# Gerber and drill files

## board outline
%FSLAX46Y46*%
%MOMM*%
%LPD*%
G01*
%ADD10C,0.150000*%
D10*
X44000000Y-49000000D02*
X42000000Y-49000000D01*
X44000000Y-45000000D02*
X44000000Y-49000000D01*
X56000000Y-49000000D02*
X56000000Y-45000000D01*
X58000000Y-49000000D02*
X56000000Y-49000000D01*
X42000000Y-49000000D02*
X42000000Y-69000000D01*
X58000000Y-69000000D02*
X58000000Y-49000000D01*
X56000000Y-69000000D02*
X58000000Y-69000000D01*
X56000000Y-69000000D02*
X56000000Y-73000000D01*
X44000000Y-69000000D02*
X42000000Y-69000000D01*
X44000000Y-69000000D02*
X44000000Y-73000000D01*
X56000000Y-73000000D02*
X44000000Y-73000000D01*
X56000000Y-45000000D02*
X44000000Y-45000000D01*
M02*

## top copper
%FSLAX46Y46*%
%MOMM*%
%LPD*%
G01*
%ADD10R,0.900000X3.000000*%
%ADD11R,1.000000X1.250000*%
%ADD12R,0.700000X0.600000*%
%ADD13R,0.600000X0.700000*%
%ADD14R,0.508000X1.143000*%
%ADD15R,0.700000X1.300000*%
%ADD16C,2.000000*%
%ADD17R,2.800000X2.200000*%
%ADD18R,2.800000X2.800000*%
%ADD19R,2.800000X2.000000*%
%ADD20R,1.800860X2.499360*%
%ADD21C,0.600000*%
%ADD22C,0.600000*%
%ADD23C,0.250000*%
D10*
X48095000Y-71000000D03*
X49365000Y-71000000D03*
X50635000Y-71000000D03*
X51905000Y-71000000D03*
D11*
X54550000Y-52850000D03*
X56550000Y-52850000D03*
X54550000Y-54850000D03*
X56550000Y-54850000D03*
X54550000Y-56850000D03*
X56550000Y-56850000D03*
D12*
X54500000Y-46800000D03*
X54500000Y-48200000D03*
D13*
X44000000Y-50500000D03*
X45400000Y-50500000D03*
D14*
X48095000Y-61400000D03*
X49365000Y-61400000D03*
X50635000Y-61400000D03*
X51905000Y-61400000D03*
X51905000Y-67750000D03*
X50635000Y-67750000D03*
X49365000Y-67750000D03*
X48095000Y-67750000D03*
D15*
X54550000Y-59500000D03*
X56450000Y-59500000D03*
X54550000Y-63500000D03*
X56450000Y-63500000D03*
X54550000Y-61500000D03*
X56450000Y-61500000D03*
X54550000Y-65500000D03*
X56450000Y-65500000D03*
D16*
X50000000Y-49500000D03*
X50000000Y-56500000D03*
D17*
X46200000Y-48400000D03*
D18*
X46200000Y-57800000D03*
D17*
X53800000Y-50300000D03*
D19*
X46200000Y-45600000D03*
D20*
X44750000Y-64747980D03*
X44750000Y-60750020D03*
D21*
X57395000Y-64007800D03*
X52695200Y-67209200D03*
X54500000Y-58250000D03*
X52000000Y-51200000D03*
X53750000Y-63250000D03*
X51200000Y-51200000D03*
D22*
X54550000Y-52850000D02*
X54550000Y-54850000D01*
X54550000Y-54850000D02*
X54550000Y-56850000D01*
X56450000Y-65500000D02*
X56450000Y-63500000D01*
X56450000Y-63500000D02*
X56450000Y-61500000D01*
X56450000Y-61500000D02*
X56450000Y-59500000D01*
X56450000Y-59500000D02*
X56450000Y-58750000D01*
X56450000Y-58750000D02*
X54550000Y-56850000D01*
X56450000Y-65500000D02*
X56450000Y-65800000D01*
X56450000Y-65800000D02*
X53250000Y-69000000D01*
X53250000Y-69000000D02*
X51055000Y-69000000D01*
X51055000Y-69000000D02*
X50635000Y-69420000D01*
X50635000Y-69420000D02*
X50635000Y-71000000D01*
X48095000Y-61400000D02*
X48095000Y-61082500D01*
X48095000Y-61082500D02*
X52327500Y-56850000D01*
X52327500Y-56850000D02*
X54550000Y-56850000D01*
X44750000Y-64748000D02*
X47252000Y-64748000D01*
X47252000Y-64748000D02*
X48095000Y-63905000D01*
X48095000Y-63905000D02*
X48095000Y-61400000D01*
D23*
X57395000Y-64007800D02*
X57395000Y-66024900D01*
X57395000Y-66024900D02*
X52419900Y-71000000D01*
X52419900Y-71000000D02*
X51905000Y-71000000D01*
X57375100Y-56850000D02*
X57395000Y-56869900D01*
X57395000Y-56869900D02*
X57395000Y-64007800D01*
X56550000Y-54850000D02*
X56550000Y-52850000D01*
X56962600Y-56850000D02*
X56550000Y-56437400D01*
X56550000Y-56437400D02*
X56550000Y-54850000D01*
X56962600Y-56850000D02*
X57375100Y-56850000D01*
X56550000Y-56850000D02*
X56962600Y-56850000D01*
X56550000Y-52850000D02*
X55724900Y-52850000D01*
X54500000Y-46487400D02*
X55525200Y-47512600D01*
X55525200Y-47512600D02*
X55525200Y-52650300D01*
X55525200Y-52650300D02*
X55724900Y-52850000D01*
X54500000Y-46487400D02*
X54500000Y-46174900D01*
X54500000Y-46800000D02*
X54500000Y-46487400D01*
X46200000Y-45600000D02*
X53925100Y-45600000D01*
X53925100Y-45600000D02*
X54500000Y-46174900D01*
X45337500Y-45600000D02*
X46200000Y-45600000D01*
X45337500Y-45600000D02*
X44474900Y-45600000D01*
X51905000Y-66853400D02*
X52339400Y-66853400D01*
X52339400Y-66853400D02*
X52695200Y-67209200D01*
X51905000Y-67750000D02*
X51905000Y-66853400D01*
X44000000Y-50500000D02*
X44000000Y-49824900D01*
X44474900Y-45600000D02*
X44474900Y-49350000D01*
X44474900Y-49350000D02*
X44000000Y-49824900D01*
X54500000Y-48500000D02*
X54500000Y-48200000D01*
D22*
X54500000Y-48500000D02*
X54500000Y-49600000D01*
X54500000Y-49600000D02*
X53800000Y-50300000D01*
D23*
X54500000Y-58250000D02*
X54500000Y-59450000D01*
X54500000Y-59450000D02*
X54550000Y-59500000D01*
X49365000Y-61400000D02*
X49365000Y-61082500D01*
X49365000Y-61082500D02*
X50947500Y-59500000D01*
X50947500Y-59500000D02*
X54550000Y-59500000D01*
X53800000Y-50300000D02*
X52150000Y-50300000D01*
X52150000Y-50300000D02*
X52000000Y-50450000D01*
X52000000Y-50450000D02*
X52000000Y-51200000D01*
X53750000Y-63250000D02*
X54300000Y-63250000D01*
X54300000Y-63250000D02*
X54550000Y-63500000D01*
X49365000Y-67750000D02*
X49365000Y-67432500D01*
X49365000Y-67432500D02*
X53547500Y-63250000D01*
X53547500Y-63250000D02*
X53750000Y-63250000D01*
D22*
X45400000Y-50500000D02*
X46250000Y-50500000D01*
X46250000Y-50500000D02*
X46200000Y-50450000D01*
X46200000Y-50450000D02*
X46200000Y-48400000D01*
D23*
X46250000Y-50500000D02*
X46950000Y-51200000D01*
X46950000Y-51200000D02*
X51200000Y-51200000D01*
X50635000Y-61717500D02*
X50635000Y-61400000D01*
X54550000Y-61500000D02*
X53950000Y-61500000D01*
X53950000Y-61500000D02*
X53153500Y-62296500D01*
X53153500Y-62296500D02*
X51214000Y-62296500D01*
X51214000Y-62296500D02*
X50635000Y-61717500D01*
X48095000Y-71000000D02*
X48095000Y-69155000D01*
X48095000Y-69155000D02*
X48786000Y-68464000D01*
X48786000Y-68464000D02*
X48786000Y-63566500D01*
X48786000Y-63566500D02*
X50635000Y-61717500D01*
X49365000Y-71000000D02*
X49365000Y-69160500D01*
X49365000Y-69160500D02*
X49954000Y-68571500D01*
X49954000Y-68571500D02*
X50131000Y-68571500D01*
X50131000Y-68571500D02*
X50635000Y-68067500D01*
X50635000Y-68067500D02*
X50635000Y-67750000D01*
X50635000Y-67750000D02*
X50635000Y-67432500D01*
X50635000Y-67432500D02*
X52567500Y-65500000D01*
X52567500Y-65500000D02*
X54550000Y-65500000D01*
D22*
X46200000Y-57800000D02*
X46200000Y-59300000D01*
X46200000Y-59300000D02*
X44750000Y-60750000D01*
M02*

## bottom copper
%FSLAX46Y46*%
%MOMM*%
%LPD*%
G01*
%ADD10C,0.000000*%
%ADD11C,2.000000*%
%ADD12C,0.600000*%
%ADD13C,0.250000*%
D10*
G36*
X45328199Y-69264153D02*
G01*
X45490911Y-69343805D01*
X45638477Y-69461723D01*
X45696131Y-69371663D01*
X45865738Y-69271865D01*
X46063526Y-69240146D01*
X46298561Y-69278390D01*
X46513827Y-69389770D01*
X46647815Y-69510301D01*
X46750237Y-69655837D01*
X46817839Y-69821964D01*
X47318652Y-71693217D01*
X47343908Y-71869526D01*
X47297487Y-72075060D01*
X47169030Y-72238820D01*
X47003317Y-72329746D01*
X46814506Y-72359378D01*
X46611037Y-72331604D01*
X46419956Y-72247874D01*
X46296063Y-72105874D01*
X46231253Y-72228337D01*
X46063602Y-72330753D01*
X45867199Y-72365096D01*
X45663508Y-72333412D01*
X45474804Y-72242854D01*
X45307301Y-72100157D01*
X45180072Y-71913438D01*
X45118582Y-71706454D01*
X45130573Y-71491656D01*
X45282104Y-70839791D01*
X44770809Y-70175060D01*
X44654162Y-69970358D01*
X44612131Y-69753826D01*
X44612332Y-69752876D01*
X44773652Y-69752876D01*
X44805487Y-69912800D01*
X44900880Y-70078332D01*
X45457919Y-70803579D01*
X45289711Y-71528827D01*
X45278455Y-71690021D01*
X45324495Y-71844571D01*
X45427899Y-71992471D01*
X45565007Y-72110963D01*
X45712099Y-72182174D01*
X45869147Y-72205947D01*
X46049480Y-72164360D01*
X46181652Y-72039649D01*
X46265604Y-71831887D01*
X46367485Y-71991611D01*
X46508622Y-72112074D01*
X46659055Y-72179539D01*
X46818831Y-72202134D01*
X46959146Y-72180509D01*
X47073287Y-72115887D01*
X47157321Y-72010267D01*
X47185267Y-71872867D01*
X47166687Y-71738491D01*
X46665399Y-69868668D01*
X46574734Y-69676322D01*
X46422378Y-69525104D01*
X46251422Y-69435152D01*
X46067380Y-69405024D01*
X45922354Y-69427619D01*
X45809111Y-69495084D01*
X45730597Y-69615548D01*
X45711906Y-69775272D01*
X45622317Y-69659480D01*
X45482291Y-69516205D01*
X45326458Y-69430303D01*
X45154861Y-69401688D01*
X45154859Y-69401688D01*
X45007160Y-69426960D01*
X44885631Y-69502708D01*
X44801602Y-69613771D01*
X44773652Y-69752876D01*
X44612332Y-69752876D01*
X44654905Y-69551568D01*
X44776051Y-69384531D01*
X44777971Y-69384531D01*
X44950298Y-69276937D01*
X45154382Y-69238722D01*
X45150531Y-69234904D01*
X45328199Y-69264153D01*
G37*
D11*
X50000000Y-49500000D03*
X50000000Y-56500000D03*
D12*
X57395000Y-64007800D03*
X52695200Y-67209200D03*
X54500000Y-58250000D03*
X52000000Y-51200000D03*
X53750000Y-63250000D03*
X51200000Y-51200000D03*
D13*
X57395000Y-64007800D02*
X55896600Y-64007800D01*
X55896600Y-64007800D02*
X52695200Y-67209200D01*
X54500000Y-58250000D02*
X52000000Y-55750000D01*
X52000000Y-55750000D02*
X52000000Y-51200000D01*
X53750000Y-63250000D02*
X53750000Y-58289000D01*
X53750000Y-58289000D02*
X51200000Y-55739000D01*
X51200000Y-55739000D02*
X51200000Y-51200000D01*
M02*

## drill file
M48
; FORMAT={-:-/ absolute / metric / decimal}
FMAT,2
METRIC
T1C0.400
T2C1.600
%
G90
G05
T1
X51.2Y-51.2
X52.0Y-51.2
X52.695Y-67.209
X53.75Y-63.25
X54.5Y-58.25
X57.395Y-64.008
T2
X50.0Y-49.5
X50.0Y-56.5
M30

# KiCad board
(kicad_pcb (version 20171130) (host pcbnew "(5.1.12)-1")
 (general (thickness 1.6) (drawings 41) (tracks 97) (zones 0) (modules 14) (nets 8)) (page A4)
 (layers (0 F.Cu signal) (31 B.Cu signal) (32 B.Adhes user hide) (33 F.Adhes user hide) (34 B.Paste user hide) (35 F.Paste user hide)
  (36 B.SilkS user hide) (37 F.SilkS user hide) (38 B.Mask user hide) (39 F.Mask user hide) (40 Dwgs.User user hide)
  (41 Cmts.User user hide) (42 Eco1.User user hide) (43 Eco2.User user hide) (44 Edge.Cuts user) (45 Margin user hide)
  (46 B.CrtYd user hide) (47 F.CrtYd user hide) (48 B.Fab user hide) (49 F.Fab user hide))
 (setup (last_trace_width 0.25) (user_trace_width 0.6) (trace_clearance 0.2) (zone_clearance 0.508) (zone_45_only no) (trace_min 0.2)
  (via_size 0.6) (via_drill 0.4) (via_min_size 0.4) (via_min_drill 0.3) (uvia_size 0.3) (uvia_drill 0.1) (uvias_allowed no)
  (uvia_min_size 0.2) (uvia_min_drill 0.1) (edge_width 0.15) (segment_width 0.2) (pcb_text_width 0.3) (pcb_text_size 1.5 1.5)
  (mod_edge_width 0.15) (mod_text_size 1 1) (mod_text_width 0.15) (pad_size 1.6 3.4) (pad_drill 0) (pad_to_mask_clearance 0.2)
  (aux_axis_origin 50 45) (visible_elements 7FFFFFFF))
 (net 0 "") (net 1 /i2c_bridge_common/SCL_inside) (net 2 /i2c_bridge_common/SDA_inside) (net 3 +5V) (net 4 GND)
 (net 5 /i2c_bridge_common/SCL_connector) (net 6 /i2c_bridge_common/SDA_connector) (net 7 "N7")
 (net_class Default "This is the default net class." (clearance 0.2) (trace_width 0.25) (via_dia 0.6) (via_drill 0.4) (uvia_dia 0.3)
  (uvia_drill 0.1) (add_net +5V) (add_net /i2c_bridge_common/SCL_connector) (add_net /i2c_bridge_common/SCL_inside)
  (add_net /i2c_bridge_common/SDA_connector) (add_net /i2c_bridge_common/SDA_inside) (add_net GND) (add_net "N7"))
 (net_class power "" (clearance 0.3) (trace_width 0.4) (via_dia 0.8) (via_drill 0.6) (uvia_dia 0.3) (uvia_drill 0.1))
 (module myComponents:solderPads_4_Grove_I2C (layer F.Cu) (at 50 71)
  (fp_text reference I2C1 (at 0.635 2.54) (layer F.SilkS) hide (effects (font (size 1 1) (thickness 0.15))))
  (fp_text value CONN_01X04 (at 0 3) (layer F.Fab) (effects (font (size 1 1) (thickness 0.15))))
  (pad 1 smd rect (at -1.905 0) (size 0.9 3) (layers F.Cu F.Paste F.Mask) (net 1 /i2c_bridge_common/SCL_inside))
  (pad 2 smd rect (at -0.635 0) (size 0.9 3) (layers F.Cu F.Paste F.Mask) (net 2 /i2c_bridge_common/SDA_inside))
  (pad 3 smd rect (at 0.635 0) (size 0.9 3) (layers F.Cu F.Paste F.Mask) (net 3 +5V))
  (pad 4 smd rect (at 1.905 0) (size 0.9 3) (layers F.Cu F.Paste F.Mask) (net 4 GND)))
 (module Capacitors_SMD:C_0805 (layer F.Cu) (at 55.55 52.85)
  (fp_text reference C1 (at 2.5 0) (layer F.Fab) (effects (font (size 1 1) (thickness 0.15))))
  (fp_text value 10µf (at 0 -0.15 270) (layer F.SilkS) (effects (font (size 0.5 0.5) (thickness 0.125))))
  (pad 1 smd rect (at -1 0) (size 1 1.25) (layers F.Cu F.Paste F.Mask) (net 3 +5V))
  (pad 2 smd rect (at 1 0) (size 1 1.25) (layers F.Cu F.Paste F.Mask) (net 4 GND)))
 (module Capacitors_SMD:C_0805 (layer F.Cu) (at 55.55 54.85)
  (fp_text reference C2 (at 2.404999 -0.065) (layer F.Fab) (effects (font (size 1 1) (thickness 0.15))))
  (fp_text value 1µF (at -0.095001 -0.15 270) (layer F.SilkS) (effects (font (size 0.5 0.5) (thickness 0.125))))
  (pad 1 smd rect (at -1 0) (size 1 1.25) (layers F.Cu F.Paste F.Mask) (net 3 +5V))
  (pad 2 smd rect (at 1 0) (size 1 1.25) (layers F.Cu F.Paste F.Mask) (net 4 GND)))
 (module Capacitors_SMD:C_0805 (layer F.Cu) (at 55.55 56.85)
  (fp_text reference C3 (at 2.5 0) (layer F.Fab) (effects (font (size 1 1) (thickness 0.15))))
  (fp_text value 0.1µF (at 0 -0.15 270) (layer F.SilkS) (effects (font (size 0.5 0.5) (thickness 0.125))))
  (pad 1 smd rect (at -1 0) (size 1 1.25) (layers F.Cu F.Paste F.Mask) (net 3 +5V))
  (pad 2 smd rect (at 1 0) (size 1 1.25) (layers F.Cu F.Paste F.Mask) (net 4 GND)))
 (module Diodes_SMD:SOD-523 (layer F.Cu) (at 54.5 47.5 90)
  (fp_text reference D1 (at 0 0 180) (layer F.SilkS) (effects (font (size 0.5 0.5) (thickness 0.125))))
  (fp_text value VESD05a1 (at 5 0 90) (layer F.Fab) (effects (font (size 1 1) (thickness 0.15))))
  (pad 2 smd rect (at 0.7 0 270) (size 0.6 0.7) (layers F.Cu F.Paste F.Mask) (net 4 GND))
  (pad 1 smd rect (at -0.7 0 270) (size 0.6 0.7) (layers F.Cu F.Paste F.Mask) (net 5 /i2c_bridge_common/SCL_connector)))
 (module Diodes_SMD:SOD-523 (layer F.Cu) (at 44.7 50.5 180)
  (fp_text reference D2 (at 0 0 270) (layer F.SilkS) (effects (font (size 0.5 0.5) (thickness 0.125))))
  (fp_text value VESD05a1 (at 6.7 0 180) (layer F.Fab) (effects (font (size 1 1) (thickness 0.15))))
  (pad 2 smd rect (at 0.7 0) (size 0.6 0.7) (layers F.Cu F.Paste F.Mask) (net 4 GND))
  (pad 1 smd rect (at -0.7 0) (size 0.6 0.7) (layers F.Cu F.Paste F.Mask) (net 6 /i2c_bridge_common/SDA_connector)))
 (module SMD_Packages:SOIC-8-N (layer F.Cu) (at 50 64.575)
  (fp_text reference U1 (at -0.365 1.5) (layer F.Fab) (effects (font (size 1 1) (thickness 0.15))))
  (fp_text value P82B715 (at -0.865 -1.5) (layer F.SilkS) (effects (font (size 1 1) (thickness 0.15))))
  (pad 8 smd rect (at -1.905 -3.175) (size 0.508 1.143) (layers F.Cu F.Paste F.Mask) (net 3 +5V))
  (pad 7 smd rect (at -0.635 -3.175) (size 0.508 1.143) (layers F.Cu F.Paste F.Mask) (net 5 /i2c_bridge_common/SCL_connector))
  (pad 6 smd rect (at 0.635 -3.175) (size 0.508 1.143) (layers F.Cu F.Paste F.Mask) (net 1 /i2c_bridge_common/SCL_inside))
  (pad 5 smd rect (at 1.905 -3.175) (size 0.508 1.143) (layers F.Cu F.Paste F.Mask))
  (pad 4 smd rect (at 1.905 3.175) (size 0.508 1.143) (layers F.Cu F.Paste F.Mask) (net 4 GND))
  (pad 3 smd rect (at 0.635 3.175) (size 0.508 1.143) (layers F.Cu F.Paste F.Mask) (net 2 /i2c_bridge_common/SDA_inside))
  (pad 2 smd rect (at -0.635 3.175) (size 0.508 1.143) (layers F.Cu F.Paste F.Mask) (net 6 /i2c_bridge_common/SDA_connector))
  (pad 1 smd rect (at -1.905 3.175) (size 0.508 1.143) (layers F.Cu F.Paste F.Mask)))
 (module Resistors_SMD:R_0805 (layer F.Cu) (at 55.5 59.5)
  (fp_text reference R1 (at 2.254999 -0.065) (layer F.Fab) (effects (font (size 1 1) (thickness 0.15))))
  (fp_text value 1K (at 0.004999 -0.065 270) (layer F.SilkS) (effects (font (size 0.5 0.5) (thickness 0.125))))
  (pad 1 smd rect (at -0.95 0) (size 0.7 1.3) (layers F.Cu F.Paste F.Mask) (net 5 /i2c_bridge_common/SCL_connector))
  (pad 2 smd rect (at 0.95 0) (size 0.7 1.3) (layers F.Cu F.Paste F.Mask) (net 3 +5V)))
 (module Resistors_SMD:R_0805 (layer F.Cu) (at 55.5 63.5)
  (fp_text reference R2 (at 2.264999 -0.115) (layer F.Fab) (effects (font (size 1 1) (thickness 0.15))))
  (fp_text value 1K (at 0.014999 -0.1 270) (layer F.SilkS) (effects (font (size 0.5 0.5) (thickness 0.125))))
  (pad 1 smd rect (at -0.95 0) (size 0.7 1.3) (layers F.Cu F.Paste F.Mask) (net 6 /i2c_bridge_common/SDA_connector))
  (pad 2 smd rect (at 0.95 0) (size 0.7 1.3) (layers F.Cu F.Paste F.Mask) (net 3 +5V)))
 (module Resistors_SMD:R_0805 (layer F.Cu) (at 55.5 61.5)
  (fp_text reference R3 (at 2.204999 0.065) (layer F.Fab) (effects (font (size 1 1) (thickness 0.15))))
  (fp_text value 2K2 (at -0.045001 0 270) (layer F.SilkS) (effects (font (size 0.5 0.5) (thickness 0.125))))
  (pad 1 smd rect (at -0.95 0) (size 0.7 1.3) (layers F.Cu F.Paste F.Mask) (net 1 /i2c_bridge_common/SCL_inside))
  (pad 2 smd rect (at 0.95 0) (size 0.7 1.3) (layers F.Cu F.Paste F.Mask) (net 3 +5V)))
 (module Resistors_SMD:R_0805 (layer F.Cu) (at 55.5 65.5)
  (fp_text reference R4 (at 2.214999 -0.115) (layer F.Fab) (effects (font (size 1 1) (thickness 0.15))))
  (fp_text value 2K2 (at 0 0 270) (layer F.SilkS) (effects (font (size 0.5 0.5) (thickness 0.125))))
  (pad 1 smd rect (at -0.95 0) (size 0.7 1.3) (layers F.Cu F.Paste F.Mask) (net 2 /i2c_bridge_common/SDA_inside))
  (pad 2 smd rect (at 0.95 0) (size 0.7 1.3) (layers F.Cu F.Paste F.Mask) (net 3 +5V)))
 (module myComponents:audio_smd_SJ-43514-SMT (layer F.Cu) (at 50 45 270)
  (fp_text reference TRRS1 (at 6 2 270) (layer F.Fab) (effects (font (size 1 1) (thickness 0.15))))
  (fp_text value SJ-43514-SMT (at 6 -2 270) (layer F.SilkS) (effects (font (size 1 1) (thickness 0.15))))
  (pad "" thru_hole circle (at 4.5 0 270) (size 2 2) (drill 1.6) (layers *.Cu *.Mask F.SilkS))
  (pad "" thru_hole circle (at 11.5 0 270) (size 2 2) (drill 1.6) (layers *.Cu *.Mask F.SilkS))
  (pad 4 smd rect (at 3.4 3.8 270) (size 2.2 2.8) (layers F.Cu F.Paste F.Mask) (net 6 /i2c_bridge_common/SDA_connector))
  (pad 2 smd rect (at 12.8 3.8 270) (size 2.8 2.8) (layers F.Cu F.Paste F.Mask) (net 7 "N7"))
  (pad 3 smd rect (at 5.3 -3.8 270) (size 2.2 2.8) (layers F.Cu F.Paste F.Mask) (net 5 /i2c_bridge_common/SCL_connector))
  (pad 1 smd rect (at 0.6 3.8 270) (size 2 2.8) (layers F.Cu F.Paste F.Mask) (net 4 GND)))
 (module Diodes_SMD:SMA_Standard (layer F.Cu) (at 44.75 62.749 90)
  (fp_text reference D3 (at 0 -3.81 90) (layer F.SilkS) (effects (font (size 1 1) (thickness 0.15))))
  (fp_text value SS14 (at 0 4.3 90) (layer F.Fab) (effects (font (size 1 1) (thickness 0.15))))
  (pad 1 smd rect (at -1.99898 0 90) (size 2.49936 1.80086) (layers F.Cu F.Paste F.Mask) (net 3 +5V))
  (pad 2 smd rect (at 1.99898 0 90) (size 2.49936 1.80086) (layers F.Cu F.Paste F.Mask) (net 7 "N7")))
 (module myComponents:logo (layer B.Cu) (at 50 70.8 180)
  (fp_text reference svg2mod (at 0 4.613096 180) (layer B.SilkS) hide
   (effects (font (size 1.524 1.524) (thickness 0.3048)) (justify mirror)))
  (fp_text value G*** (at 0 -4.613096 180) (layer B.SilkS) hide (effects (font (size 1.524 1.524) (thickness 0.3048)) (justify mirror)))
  (fp_poly
   (pts (xy 4.849469 1.565096) (xy 4.269403 1.184452) (xy 4.288094 1.024728) (xy 4.377683 1.14052) (xy 4.517709 1.283795)
    (xy 4.673542 1.369697) (xy 4.845139 1.398312) (xy 4.845141 1.398312) (xy 4.99284 1.37304) (xy 5.114369 1.297292) (xy 5.198398 1.186229)
    (xy 5.226348 1.047124) (xy 5.194513 0.8872) (xy 5.09912 0.721668) (xy 4.542081 -0.003579) (xy 4.710289 -0.728827)
    (xy 4.721545 -0.890021) (xy 4.675505 -1.044571) (xy 4.572101 -1.192471) (xy 4.434993 -1.310963) (xy 4.287901 -1.382174)
    (xy 4.130853 -1.405947) (xy 3.95052 -1.36436) (xy 3.818348 -1.239649) (xy 3.734396 -1.031887) (xy 3.632515 -1.191611)
    (xy 3.491378 -1.312074) (xy 3.340945 -1.379539) (xy 3.181169 -1.402134) (xy 3.040854 -1.380509) (xy 2.926713 -1.315887)
    (xy 2.842679 -1.210267) (xy 2.814733 -1.072867) (xy 2.833313 -0.938491) (xy 3.334601 0.931332) (xy 3.425266 1.123678)
    (xy 3.577622 1.274896) (xy 3.748578 1.364848) (xy 3.93262 1.394976) (xy 4.077646 1.372381) (xy 4.190889 1.304916) (xy 4.269403 1.184452)
    (xy 4.849469 1.565096) (xy 4.671801 1.535847) (xy 4.509089 1.456195) (xy 4.361523 1.338277) (xy 4.303869 1.428337)
    (xy 4.134262 1.528135) (xy 3.936474 1.559854) (xy 3.701439 1.52161) (xy 3.486173 1.41023) (xy 3.352185 1.289699) (xy 3.249763 1.144163)
    (xy 3.182161 0.978036) (xy 2.681348 -0.893217) (xy 2.656092 -1.069526) (xy 2.702513 -1.27506) (xy 2.83097 -1.43882)
    (xy 2.996683 -1.529746) (xy 3.185494 -1.559378) (xy 3.388963 -1.531604) (xy 3.580044 -1.447874) (xy 3.703937 -1.305874)
    (xy 3.768747 -1.428337) (xy 3.936398 -1.530753) (xy 4.132801 -1.565096) (xy 4.336492 -1.533412) (xy 4.525196 -1.442854)
    (xy 4.692699 -1.300157) (xy 4.819928 -1.113438) (xy 4.881418 -0.906454) (xy 4.869427 -0.691656) (xy 4.717896 -0.039791)
    (xy 5.229191 0.62494) (xy 5.345838 0.829642) (xy 5.387869 1.046174) (xy 5.345095 1.248432) (xy 5.223949 1.415469) (xy 5.222029 1.415469)
    (xy 5.049702 1.523063) (xy 4.845618 1.561278) (xy 4.849469 1.565096))
   (layer B.Cu) (width 0)))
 (gr_line (start 44 49) (end 42 49) (layer Edge.Cuts) (width 0.15))
 (gr_line (start 44 45) (end 44 49) (layer Edge.Cuts) (width 0.15))
 (gr_line (start 56 49) (end 56 45) (layer Edge.Cuts) (width 0.15))
 (gr_line (start 58 49) (end 56 49) (layer Edge.Cuts) (width 0.15))
 (gr_line (start 42 49) (end 42 69) (layer Edge.Cuts) (width 0.15))
 (gr_line (start 58 69) (end 58 49) (layer Edge.Cuts) (width 0.15))
 (gr_line (start 56 69) (end 58 69) (layer Edge.Cuts) (width 0.15))
 (gr_line (start 56 69) (end 56 73) (layer Edge.Cuts) (width 0.15))
 (gr_line (start 44 69) (end 42 69) (layer Edge.Cuts) (width 0.15))
 (gr_line (start 44 69) (end 44 73) (layer Edge.Cuts) (width 0.15))
 (gr_line (start 56 73) (end 44 73) (layer Edge.Cuts) (width 0.15))
 (gr_line (start 56 45) (end 44 45) (layer Edge.Cuts) (width 0.15))
 (segment (start 54.55 52.85) (end 54.55 54.85) (width 0.6) (layer F.Cu) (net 3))
 (segment (start 54.55 54.85) (end 54.55 56.85) (width 0.6) (layer F.Cu) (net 3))
 (segment (start 56.45 65.5) (end 56.45 63.5) (width 0.6) (layer F.Cu) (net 3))
 (segment (start 56.45 63.5) (end 56.45 61.5) (width 0.6) (layer F.Cu) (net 3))
 (segment (start 56.45 61.5) (end 56.45 59.5) (width 0.6) (layer F.Cu) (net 3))
 (segment (start 56.45 59.5) (end 56.45 58.75) (width 0.6) (layer F.Cu) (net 3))
 (segment (start 56.45 58.75) (end 54.55 56.85) (width 0.6) (layer F.Cu) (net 3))
 (segment (start 56.45 65.5) (end 56.45 65.8) (width 0.6) (layer F.Cu) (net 3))
 (segment (start 56.45 65.8) (end 53.25 69) (width 0.6) (layer F.Cu) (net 3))
 (segment (start 53.25 69) (end 51.055 69) (width 0.6) (layer F.Cu) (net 3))
 (segment (start 51.055 69) (end 50.635 69.42) (width 0.6) (layer F.Cu) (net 3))
 (segment (start 50.635 69.42) (end 50.635 71) (width 0.6) (layer F.Cu) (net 3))
 (segment (start 48.095 61.4) (end 48.095 61.0825) (width 0.6) (layer F.Cu) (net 3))
 (segment (start 48.095 61.0825) (end 52.3275 56.85) (width 0.6) (layer F.Cu) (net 3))
 (segment (start 52.3275 56.85) (end 54.55 56.85) (width 0.6) (layer F.Cu) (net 3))
 (segment (start 44.75 64.748) (end 47.252 64.748) (width 0.6) (layer F.Cu) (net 3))
 (segment (start 47.252 64.748) (end 48.095 63.905) (width 0.6) (layer F.Cu) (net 3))
 (segment (start 48.095 63.905) (end 48.095 61.4) (width 0.6) (layer F.Cu) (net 3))
 (segment (start 57.395 64.0078) (end 57.395 66.0249) (width 0.25) (layer F.Cu) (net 4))
 (segment (start 57.395 66.0249) (end 52.4199 71) (width 0.25) (layer F.Cu) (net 4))
 (segment (start 52.4199 71) (end 51.905 71) (width 0.25) (layer F.Cu) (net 4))
 (segment (start 57.3751 56.85) (end 57.395 56.8699) (width 0.25) (layer F.Cu) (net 4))
 (segment (start 57.395 56.8699) (end 57.395 64.0078) (width 0.25) (layer F.Cu) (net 4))
 (segment (start 56.55 54.85) (end 56.55 52.85) (width 0.25) (layer F.Cu) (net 4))
 (segment (start 56.9626 56.85) (end 56.55 56.4374) (width 0.25) (layer F.Cu) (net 4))
 (segment (start 56.55 56.4374) (end 56.55 54.85) (width 0.25) (layer F.Cu) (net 4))
 (segment (start 56.9626 56.85) (end 57.3751 56.85) (width 0.25) (layer F.Cu) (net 4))
 (segment (start 56.55 56.85) (end 56.9626 56.85) (width 0.25) (layer F.Cu) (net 4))
 (segment (start 56.55 52.85) (end 55.7249 52.85) (width 0.25) (layer F.Cu) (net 4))
 (segment (start 54.5 46.4874) (end 55.5252 47.5126) (width 0.25) (layer F.Cu) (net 4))
 (segment (start 55.5252 47.5126) (end 55.5252 52.6503) (width 0.25) (layer F.Cu) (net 4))
 (segment (start 55.5252 52.6503) (end 55.7249 52.85) (width 0.25) (layer F.Cu) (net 4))
 (segment (start 54.5 46.4874) (end 54.5 46.1749) (width 0.25) (layer F.Cu) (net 4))
 (segment (start 54.5 46.8) (end 54.5 46.4874) (width 0.25) (layer F.Cu) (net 4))
 (segment (start 46.2 45.6) (end 53.9251 45.6) (width 0.25) (layer F.Cu) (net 4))
 (segment (start 53.9251 45.6) (end 54.5 46.1749) (width 0.25) (layer F.Cu) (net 4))
 (segment (start 45.3375 45.6) (end 46.2 45.6) (width 0.25) (layer F.Cu) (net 4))
 (segment (start 45.3375 45.6) (end 44.4749 45.6) (width 0.25) (layer F.Cu) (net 4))
 (segment (start 51.905 66.8534) (end 52.3394 66.8534) (width 0.25) (layer F.Cu) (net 4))
 (segment (start 52.3394 66.8534) (end 52.6952 67.2092) (width 0.25) (layer F.Cu) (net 4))
 (segment (start 57.395 64.0078) (end 55.8966 64.0078) (width 0.25) (layer B.Cu) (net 4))
 (segment (start 55.8966 64.0078) (end 52.6952 67.2092) (width 0.25) (layer B.Cu) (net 4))
 (segment (start 51.905 67.75) (end 51.905 66.8534) (width 0.25) (layer F.Cu) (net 4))
 (segment (start 44 50.5) (end 44 49.8249) (width 0.25) (layer F.Cu) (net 4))
 (segment (start 44.4749 45.6) (end 44.4749 49.35) (width 0.25) (layer F.Cu) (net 4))
 (segment (start 44.4749 49.35) (end 44 49.8249) (width 0.25) (layer F.Cu) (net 4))
 (via (at 57.395 64.0078) (size 0.6) (layers F.Cu B.Cu) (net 4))
 (via (at 52.6952 67.2092) (size 0.6) (layers F.Cu B.Cu) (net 4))
 (segment (start 54.5 48.5) (end 54.5 48.2) (width 0.25) (layer F.Cu) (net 5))
 (segment (start 54.5 48.5) (end 54.5 49.6) (width 0.6) (layer F.Cu) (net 5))
 (segment (start 54.5 49.6) (end 53.8 50.3) (width 0.6) (layer F.Cu) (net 5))
 (segment (start 54.5 58.25) (end 54.5 59.45) (width 0.25) (layer F.Cu) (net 5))
 (segment (start 54.5 59.45) (end 54.55 59.5) (width 0.25) (layer F.Cu) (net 5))
 (segment (start 49.365 61.4) (end 49.365 61.0825) (width 0.25) (layer F.Cu) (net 5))
 (segment (start 49.365 61.0825) (end 50.9475 59.5) (width 0.25) (layer F.Cu) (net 5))
 (segment (start 50.9475 59.5) (end 54.55 59.5) (width 0.25) (layer F.Cu) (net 5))
 (segment (start 53.8 50.3) (end 52.15 50.3) (width 0.25) (layer F.Cu) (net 5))
 (segment (start 52.15 50.3) (end 52 50.45) (width 0.25) (layer F.Cu) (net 5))
 (segment (start 52 50.45) (end 52 51.2) (width 0.25) (layer F.Cu) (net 5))
 (segment (start 54.5 58.25) (end 52 55.75) (width 0.25) (layer B.Cu) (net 5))
 (segment (start 52 55.75) (end 52 51.2) (width 0.25) (layer B.Cu) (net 5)) (via (at 54.5 58.25) (size 0.6) (layers F.Cu B.Cu) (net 5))
 (via (at 52 51.2) (size 0.6) (layers F.Cu B.Cu) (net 5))
 (segment (start 53.75 63.25) (end 54.3 63.25) (width 0.25) (layer F.Cu) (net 6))
 (segment (start 54.3 63.25) (end 54.55 63.5) (width 0.25) (layer F.Cu) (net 6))
 (segment (start 49.365 67.75) (end 49.365 67.4325) (width 0.25) (layer F.Cu) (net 6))
 (segment (start 49.365 67.4325) (end 53.5475 63.25) (width 0.25) (layer F.Cu) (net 6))
 (segment (start 53.5475 63.25) (end 53.75 63.25) (width 0.25) (layer F.Cu) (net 6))
 (segment (start 45.4 50.5) (end 46.25 50.5) (width 0.6) (layer F.Cu) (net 6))
 (segment (start 46.25 50.5) (end 46.2 50.45) (width 0.6) (layer F.Cu) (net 6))
 (segment (start 46.2 50.45) (end 46.2 48.4) (width 0.6) (layer F.Cu) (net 6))
 (segment (start 53.75 63.25) (end 53.75 58.289) (width 0.25) (layer B.Cu) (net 6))
 (segment (start 53.75 58.289) (end 51.2 55.739) (width 0.25) (layer B.Cu) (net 6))
 (segment (start 51.2 55.739) (end 51.2 51.2) (width 0.25) (layer B.Cu) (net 6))
 (segment (start 46.25 50.5) (end 46.95 51.2) (width 0.25) (layer F.Cu) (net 6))
 (segment (start 46.95 51.2) (end 51.2 51.2) (width 0.25) (layer F.Cu) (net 6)) (via (at 53.75 63.25) (size 0.6) (layers F.Cu B.Cu) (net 6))
 (via (at 51.2 51.2) (size 0.6) (layers F.Cu B.Cu) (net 6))
 (segment (start 50.635 61.7175) (end 50.635 61.4) (width 0.25) (layer F.Cu) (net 1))
 (segment (start 54.55 61.5) (end 53.95 61.5) (width 0.25) (layer F.Cu) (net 1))
 (segment (start 53.95 61.5) (end 53.1535 62.2965) (width 0.25) (layer F.Cu) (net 1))
 (segment (start 53.1535 62.2965) (end 51.214 62.2965) (width 0.25) (layer F.Cu) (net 1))
 (segment (start 51.214 62.2965) (end 50.635 61.7175) (width 0.25) (layer F.Cu) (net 1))
 (segment (start 48.095 71) (end 48.095 69.155) (width 0.25) (layer F.Cu) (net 1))
 (segment (start 48.095 69.155) (end 48.786 68.464) (width 0.25) (layer F.Cu) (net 1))
 (segment (start 48.786 68.464) (end 48.786 63.5665) (width 0.25) (layer F.Cu) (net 1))
 (segment (start 48.786 63.5665) (end 50.635 61.7175) (width 0.25) (layer F.Cu) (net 1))
 (segment (start 49.365 71) (end 49.365 69.1605) (width 0.25) (layer F.Cu) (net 2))
 (segment (start 49.365 69.1605) (end 49.954 68.5715) (width 0.25) (layer F.Cu) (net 2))
 (segment (start 49.954 68.5715) (end 50.131 68.5715) (width 0.25) (layer F.Cu) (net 2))
 (segment (start 50.131 68.5715) (end 50.635 68.0675) (width 0.25) (layer F.Cu) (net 2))
 (segment (start 50.635 68.0675) (end 50.635 67.75) (width 0.25) (layer F.Cu) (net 2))
 (segment (start 50.635 67.75) (end 50.635 67.4325) (width 0.25) (layer F.Cu) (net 2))
 (segment (start 50.635 67.4325) (end 52.5675 65.5) (width 0.25) (layer F.Cu) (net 2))
 (segment (start 52.5675 65.5) (end 54.55 65.5) (width 0.25) (layer F.Cu) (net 2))
 (segment (start 46.2 57.8) (end 46.2 59.3) (width 0.6) (layer F.Cu) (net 7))
 (segment (start 46.2 59.3) (end 44.75 60.75) (width 0.6) (layer F.Cu) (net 7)))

